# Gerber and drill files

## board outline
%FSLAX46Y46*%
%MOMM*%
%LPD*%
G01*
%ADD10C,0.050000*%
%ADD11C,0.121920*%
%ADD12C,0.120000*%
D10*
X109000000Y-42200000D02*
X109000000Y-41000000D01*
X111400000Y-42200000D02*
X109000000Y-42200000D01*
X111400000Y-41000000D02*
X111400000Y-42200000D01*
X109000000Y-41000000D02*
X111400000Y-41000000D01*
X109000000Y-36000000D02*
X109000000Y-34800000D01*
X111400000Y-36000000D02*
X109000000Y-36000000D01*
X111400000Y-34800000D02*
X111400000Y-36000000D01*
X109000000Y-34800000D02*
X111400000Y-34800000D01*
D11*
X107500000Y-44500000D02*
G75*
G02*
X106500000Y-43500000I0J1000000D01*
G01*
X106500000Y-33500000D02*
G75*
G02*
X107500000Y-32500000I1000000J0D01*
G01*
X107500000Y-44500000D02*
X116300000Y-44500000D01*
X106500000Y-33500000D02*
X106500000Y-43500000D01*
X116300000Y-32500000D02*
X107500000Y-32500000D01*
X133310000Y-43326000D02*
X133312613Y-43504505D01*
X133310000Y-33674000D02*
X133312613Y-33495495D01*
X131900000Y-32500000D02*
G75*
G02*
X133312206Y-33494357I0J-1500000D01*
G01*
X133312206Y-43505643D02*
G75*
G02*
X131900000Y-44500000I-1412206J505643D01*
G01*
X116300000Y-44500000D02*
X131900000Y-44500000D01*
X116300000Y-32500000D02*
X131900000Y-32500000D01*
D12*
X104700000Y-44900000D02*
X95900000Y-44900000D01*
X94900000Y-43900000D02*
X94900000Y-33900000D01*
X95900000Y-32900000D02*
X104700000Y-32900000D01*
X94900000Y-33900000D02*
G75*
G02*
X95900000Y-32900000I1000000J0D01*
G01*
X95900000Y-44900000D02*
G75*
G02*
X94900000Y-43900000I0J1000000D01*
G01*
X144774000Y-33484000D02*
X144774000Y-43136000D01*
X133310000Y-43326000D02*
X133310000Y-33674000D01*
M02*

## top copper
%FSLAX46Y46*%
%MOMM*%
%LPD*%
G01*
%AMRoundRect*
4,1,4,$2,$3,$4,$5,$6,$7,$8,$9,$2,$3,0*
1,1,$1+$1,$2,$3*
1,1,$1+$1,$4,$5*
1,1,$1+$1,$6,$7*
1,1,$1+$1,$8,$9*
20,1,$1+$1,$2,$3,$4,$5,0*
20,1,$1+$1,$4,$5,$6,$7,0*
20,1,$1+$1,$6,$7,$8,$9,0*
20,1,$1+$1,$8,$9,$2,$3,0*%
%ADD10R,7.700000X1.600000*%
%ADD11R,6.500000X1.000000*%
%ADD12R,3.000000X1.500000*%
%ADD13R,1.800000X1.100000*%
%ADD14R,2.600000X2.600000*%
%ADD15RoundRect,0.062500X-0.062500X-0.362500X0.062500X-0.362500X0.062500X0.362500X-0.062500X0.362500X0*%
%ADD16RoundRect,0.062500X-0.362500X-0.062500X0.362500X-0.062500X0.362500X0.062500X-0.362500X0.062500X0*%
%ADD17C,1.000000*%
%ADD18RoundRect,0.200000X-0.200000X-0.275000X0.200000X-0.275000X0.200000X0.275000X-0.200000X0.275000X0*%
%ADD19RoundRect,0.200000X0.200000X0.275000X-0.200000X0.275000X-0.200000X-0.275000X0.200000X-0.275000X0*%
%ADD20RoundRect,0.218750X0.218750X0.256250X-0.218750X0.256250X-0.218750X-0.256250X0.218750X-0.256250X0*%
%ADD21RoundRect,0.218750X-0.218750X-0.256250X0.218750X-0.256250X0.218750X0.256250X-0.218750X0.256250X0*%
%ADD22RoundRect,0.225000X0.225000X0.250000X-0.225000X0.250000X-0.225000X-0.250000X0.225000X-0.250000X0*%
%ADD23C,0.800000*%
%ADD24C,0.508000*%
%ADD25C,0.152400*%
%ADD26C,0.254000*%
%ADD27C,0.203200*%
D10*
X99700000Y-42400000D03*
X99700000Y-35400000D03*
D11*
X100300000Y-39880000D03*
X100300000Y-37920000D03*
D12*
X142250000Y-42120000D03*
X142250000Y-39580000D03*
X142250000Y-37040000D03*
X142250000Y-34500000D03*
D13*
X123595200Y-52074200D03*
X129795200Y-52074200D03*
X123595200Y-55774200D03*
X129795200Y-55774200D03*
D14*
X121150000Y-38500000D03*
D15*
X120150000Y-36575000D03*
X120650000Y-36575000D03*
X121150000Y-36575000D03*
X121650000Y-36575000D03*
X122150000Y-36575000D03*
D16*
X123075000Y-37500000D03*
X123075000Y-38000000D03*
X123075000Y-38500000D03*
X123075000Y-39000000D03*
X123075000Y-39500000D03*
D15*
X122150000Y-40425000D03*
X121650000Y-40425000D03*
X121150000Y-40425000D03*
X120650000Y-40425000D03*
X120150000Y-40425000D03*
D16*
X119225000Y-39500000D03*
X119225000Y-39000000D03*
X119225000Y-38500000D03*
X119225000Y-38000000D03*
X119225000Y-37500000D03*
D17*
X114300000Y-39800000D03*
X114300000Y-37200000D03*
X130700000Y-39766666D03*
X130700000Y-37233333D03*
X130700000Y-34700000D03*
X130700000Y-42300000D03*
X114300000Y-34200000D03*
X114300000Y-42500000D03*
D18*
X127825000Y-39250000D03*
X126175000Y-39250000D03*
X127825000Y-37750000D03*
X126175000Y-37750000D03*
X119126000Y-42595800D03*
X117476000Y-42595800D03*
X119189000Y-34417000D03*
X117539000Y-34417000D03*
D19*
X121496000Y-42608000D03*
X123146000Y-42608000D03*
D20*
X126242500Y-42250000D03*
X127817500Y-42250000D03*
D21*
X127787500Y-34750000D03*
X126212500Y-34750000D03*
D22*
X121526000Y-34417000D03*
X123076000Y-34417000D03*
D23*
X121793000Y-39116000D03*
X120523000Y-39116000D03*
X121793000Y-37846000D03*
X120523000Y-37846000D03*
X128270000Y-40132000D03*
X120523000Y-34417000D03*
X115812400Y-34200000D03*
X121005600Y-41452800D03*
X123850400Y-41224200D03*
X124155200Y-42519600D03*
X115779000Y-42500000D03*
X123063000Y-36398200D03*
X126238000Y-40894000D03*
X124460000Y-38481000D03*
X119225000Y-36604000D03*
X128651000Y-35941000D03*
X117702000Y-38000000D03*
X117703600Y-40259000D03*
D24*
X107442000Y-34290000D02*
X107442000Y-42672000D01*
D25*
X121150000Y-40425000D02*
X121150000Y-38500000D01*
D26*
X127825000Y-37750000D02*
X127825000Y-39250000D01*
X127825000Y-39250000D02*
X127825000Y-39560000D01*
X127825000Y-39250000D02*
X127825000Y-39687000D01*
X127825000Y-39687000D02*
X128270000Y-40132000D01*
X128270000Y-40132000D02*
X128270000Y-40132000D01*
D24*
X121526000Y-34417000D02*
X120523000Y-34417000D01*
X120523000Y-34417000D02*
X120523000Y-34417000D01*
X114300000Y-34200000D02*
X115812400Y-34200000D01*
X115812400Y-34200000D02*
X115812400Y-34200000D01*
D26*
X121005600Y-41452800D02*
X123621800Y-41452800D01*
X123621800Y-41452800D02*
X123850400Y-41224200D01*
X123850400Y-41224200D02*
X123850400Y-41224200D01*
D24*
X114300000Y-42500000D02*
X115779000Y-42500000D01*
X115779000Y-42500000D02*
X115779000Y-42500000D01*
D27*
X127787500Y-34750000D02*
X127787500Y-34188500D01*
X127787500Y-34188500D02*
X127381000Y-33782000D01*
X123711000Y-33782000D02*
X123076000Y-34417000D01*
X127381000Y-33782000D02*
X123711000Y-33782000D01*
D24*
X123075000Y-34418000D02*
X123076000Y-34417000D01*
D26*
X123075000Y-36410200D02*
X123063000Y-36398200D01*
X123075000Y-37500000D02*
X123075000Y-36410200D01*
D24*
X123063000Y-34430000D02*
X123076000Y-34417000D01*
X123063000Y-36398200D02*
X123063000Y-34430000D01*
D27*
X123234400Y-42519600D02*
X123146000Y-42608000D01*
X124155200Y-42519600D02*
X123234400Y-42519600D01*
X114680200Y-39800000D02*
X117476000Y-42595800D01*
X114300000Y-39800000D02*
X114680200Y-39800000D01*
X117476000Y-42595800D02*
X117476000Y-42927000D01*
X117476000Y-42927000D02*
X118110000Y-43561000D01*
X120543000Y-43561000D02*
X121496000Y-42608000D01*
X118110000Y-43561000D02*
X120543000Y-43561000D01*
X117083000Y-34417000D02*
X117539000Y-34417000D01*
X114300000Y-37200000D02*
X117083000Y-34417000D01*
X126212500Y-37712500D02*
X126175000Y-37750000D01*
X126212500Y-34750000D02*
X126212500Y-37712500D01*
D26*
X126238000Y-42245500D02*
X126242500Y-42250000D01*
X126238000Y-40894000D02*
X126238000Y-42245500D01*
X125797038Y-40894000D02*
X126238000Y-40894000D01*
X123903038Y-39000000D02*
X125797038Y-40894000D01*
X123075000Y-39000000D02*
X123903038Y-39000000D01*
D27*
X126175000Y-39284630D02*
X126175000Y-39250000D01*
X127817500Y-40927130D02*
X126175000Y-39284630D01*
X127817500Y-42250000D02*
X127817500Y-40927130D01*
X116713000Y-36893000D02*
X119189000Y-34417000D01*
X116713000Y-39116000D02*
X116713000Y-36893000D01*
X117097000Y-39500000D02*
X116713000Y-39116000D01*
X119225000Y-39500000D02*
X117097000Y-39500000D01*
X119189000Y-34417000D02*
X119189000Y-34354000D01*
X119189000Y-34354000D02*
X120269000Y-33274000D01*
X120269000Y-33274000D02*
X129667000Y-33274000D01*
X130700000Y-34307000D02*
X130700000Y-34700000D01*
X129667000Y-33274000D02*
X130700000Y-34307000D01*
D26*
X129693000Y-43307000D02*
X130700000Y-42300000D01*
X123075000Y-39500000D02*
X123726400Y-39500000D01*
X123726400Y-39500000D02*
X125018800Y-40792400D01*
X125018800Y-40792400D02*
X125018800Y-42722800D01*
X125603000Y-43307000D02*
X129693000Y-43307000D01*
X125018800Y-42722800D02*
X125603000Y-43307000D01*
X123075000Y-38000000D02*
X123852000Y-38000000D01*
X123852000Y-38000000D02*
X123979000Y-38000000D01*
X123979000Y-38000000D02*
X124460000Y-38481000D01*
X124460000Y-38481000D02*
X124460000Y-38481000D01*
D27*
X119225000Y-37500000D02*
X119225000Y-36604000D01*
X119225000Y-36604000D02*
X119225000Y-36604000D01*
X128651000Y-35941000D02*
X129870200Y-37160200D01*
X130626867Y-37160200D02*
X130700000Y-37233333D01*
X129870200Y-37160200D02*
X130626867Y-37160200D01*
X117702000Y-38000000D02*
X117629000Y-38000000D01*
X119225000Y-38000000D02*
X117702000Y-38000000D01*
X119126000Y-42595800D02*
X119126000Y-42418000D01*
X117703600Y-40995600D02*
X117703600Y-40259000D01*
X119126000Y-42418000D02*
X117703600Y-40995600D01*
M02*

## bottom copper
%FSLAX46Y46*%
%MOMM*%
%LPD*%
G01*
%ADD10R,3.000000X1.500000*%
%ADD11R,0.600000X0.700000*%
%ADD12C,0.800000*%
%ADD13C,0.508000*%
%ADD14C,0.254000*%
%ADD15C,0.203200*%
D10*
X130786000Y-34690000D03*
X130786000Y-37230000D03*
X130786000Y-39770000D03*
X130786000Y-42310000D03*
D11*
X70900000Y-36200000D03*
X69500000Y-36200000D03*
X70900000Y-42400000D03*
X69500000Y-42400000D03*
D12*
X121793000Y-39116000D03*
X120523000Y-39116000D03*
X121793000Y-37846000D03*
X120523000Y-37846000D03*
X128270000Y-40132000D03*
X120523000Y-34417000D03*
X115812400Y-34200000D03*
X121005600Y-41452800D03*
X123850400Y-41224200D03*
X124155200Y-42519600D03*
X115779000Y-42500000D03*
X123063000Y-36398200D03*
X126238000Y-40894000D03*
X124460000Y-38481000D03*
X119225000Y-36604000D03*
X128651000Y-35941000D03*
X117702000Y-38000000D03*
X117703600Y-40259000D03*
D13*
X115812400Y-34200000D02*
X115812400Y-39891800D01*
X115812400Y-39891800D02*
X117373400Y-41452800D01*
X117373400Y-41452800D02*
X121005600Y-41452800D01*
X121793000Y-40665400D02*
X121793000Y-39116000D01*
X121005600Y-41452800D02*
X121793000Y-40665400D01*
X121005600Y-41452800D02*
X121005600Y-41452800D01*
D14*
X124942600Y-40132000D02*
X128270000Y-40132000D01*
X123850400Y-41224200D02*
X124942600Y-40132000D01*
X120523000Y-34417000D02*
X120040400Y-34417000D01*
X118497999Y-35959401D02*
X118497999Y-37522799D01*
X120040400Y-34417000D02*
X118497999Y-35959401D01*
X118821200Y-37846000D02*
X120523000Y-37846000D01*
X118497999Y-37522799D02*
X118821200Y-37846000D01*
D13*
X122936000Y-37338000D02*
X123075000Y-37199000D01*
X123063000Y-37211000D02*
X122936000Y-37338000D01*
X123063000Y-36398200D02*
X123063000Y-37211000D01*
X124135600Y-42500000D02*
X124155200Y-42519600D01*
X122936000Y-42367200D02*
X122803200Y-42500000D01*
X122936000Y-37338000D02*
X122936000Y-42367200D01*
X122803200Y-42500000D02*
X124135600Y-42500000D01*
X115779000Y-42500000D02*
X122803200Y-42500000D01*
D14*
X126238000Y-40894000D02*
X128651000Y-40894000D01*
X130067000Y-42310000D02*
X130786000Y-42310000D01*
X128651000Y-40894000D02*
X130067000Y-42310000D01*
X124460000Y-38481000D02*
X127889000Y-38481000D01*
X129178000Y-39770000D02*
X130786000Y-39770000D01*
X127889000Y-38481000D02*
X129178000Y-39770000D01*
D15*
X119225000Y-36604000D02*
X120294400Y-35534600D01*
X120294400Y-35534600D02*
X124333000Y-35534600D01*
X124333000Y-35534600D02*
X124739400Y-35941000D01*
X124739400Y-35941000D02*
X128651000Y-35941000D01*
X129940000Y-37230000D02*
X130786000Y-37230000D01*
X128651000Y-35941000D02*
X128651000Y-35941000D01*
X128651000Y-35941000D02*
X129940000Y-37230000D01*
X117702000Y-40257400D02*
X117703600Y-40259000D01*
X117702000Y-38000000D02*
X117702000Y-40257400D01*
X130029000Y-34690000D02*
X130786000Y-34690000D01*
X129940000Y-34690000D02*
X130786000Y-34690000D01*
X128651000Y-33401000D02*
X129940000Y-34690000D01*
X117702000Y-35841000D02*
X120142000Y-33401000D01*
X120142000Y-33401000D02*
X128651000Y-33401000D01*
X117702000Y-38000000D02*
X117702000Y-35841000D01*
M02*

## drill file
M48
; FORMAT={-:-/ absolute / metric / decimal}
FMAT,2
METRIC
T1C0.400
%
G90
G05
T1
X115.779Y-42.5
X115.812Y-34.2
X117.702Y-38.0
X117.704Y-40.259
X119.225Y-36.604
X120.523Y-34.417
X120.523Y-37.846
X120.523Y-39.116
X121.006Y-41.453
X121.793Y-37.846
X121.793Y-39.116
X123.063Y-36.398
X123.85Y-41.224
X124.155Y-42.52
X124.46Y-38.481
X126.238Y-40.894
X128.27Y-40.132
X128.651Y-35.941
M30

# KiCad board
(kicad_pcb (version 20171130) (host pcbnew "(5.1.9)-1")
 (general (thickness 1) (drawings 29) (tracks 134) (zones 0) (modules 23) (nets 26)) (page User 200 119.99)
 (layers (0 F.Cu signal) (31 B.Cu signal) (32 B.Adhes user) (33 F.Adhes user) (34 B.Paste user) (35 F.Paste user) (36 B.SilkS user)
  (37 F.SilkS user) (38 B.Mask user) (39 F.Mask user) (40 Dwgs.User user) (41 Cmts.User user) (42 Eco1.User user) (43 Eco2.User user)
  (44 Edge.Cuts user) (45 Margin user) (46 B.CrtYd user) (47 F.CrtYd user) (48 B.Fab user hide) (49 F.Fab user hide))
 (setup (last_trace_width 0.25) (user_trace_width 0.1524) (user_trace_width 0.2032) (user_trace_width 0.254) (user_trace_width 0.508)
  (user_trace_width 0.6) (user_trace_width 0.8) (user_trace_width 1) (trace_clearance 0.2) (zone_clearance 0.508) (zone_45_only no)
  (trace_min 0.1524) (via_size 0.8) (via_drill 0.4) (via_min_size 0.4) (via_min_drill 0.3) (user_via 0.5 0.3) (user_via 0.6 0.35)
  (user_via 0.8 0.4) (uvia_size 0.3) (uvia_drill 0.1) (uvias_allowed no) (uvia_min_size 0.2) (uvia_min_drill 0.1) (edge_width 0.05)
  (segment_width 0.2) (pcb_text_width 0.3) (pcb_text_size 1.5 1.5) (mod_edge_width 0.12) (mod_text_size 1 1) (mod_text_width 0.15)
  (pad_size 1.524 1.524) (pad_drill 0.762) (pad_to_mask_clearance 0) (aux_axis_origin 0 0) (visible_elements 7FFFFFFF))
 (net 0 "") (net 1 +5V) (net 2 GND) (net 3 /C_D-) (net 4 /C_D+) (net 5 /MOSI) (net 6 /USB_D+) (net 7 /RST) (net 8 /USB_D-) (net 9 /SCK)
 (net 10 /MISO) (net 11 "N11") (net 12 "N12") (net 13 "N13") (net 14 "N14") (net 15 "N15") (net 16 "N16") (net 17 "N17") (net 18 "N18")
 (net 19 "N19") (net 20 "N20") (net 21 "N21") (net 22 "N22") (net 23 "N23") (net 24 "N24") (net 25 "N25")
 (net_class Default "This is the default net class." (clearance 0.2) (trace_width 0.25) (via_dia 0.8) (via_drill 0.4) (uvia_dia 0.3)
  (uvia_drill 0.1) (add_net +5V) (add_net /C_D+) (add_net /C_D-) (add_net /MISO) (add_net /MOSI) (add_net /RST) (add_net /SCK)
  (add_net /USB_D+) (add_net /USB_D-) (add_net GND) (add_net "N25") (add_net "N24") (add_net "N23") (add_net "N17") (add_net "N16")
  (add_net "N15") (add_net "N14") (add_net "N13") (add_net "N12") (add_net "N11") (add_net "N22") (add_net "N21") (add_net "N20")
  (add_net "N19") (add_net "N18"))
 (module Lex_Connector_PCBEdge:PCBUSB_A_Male (layer F.Cu) (at 100.7 38.9 180)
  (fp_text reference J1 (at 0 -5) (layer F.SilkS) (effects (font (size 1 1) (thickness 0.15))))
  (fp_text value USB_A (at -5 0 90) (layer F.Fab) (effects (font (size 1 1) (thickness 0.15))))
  (fp_line (start -4 -6) (end 4.8 -6) (layer Edge.Cuts) (width 0.12))
  (fp_line (start 5.8 -5) (end 5.8 5) (layer Edge.Cuts) (width 0.12))
  (fp_line (start 4.8 6) (end -4 6) (layer Edge.Cuts) (width 0.12))
  (fp_arc (start 4.8 5) (end 4.8 6) (angle -90) (layer Edge.Cuts) (width 0.12))
  (fp_arc (start 4.8 -5) (end 5.8 -5) (angle -90) (layer Edge.Cuts) (width 0.12))
  (pad 1 connect rect (at 1 -3.5 180) (size 7.7 1.6) (layers F.Cu F.Mask) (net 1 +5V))
  (pad 4 connect rect (at 1 3.5 180) (size 7.7 1.6) (layers F.Cu F.Mask) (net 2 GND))
  (pad 2 connect rect (at 0.4 -0.98 180) (size 6.5 1) (layers F.Cu F.Mask) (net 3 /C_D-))
  (pad 3 connect rect (at 0.4 0.98 180) (size 6.5 1) (layers F.Cu F.Mask) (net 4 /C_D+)))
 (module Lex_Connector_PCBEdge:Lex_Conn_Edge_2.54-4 (layer F.Cu) (at 139.964 38.31)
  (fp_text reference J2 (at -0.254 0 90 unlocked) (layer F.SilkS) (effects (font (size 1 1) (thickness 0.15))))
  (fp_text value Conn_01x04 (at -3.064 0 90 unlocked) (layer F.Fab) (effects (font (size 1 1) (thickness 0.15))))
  (fp_line (start 4.81 -4.826) (end 4.81 4.826) (layer Edge.Cuts) (width 0.12))
  (pad 4 smd rect (at 2.286 3.81 270) (size 1.5 3) (layers F.Cu F.Paste F.Mask) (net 1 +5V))
  (pad 3 smd rect (at 2.286 1.27 270) (size 1.5 3) (layers F.Cu F.Paste F.Mask) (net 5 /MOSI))
  (pad 2 smd rect (at 2.286 -1.27 270) (size 1.5 3) (layers F.Cu F.Paste F.Mask) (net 2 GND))
  (pad 1 smd rect (at 2.286 -3.81 270) (size 1.5 3) (layers F.Cu F.Paste F.Mask) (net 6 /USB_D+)))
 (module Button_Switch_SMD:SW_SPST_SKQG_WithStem (layer F.Cu) (at 126.6952 53.9242 180)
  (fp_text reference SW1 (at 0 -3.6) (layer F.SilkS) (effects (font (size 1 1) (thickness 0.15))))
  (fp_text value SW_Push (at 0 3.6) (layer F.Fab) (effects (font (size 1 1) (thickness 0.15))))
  (pad 2 smd rect (at 3.1 1.85 180) (size 1.8 1.1) (layers F.Cu F.Paste F.Mask) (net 2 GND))
  (pad 2 smd rect (at -3.1 1.85 180) (size 1.8 1.1) (layers F.Cu F.Paste F.Mask) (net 2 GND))
  (pad 1 smd rect (at 3.1 -1.85 180) (size 1.8 1.1) (layers F.Cu F.Paste F.Mask) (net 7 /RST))
  (pad 1 smd rect (at -3.1 -1.85 180) (size 1.8 1.1) (layers F.Cu F.Paste F.Mask) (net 7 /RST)))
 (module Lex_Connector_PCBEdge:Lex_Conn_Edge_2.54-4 (layer B.Cu) (at 128.5 38.5)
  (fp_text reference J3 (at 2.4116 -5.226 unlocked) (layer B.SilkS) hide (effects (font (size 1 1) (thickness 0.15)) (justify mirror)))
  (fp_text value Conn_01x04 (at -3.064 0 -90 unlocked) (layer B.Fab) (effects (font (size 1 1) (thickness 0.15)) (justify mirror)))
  (fp_line (start 4.81 4.826) (end 4.81 -4.826) (layer Edge.Cuts) (width 0.12))
  (pad 4 smd rect (at 2.286 -3.81 90) (size 1.5 3) (layers B.Cu B.Paste B.Mask) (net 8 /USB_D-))
  (pad 3 smd rect (at 2.286 -1.27 90) (size 1.5 3) (layers B.Cu B.Paste B.Mask) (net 7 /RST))
  (pad 2 smd rect (at 2.286 1.27 90) (size 1.5 3) (layers B.Cu B.Paste B.Mask) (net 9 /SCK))
  (pad 1 smd rect (at 2.286 3.81 90) (size 1.5 3) (layers B.Cu B.Paste B.Mask) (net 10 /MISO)))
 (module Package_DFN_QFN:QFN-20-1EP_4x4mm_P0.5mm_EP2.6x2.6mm (layer F.Cu) (at 121.15 38.5)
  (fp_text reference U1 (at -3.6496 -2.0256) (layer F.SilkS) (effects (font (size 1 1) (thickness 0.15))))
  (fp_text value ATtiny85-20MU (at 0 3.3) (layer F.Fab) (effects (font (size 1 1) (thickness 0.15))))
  (pad "" smd roundrect (at 0.65 0.65) (size 1.05 1.05) (layers F.Paste) (roundrect_rratio 0.238095))
  (pad "" smd roundrect (at 0.65 -0.65) (size 1.05 1.05) (layers F.Paste) (roundrect_rratio 0.238095))
  (pad "" smd roundrect (at -0.65 0.65) (size 1.05 1.05) (layers F.Paste) (roundrect_rratio 0.238095))
  (pad "" smd roundrect (at -0.65 -0.65) (size 1.05 1.05) (layers F.Paste) (roundrect_rratio 0.238095))
  (pad 21 smd rect (at 0 0) (size 2.6 2.6) (layers F.Cu F.Mask) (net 2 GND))
  (pad 20 smd roundrect (at -1 -1.925) (size 0.25 0.85) (layers F.Cu F.Paste F.Mask) (roundrect_rratio 0.25) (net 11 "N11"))
  (pad 19 smd roundrect (at -0.5 -1.925) (size 0.25 0.85) (layers F.Cu F.Paste F.Mask) (roundrect_rratio 0.25) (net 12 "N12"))
  (pad 18 smd roundrect (at 0 -1.925) (size 0.25 0.85) (layers F.Cu F.Paste F.Mask) (roundrect_rratio 0.25) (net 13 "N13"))
  (pad 17 smd roundrect (at 0.5 -1.925) (size 0.25 0.85) (layers F.Cu F.Paste F.Mask) (roundrect_rratio 0.25) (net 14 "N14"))
  (pad 16 smd roundrect (at 1 -1.925) (size 0.25 0.85) (layers F.Cu F.Paste F.Mask) (roundrect_rratio 0.25) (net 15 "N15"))
  (pad 15 smd roundrect (at 1.925 -1) (size 0.85 0.25) (layers F.Cu F.Paste F.Mask) (roundrect_rratio 0.25) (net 1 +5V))
  (pad 14 smd roundrect (at 1.925 -0.5) (size 0.85 0.25) (layers F.Cu F.Paste F.Mask) (roundrect_rratio 0.25) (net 9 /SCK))
  (pad 13 smd roundrect (at 1.925 0) (size 0.85 0.25) (layers F.Cu F.Paste F.Mask) (roundrect_rratio 0.25) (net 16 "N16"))
  (pad 12 smd roundrect (at 1.925 0.5) (size 0.85 0.25) (layers F.Cu F.Paste F.Mask) (roundrect_rratio 0.25) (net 10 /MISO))
  (pad 11 smd roundrect (at 1.925 1) (size 0.85 0.25) (layers F.Cu F.Paste F.Mask) (roundrect_rratio 0.25) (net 5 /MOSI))
  (pad 10 smd roundrect (at 1 1.925) (size 0.25 0.85) (layers F.Cu F.Paste F.Mask) (roundrect_rratio 0.25) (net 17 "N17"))
  (pad 9 smd roundrect (at 0.5 1.925) (size 0.25 0.85) (layers F.Cu F.Paste F.Mask) (roundrect_rratio 0.25) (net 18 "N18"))
  (pad 8 smd roundrect (at 0 1.925) (size 0.25 0.85) (layers F.Cu F.Paste F.Mask) (roundrect_rratio 0.25) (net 2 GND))
  (pad 7 smd roundrect (at -0.5 1.925) (size 0.25 0.85) (layers F.Cu F.Paste F.Mask) (roundrect_rratio 0.25) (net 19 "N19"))
  (pad 6 smd roundrect (at -1 1.925) (size 0.25 0.85) (layers F.Cu F.Paste F.Mask) (roundrect_rratio 0.25) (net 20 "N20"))
  (pad 5 smd roundrect (at -1.925 1) (size 0.85 0.25) (layers F.Cu F.Paste F.Mask) (roundrect_rratio 0.25) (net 6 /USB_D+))
  (pad 4 smd roundrect (at -1.925 0.5) (size 0.85 0.25) (layers F.Cu F.Paste F.Mask) (roundrect_rratio 0.25) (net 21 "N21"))
  (pad 3 smd roundrect (at -1.925 0) (size 0.85 0.25) (layers F.Cu F.Paste F.Mask) (roundrect_rratio 0.25) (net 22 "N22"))
  (pad 2 smd roundrect (at -1.925 -0.5) (size 0.85 0.25) (layers F.Cu F.Paste F.Mask) (roundrect_rratio 0.25) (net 8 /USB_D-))
  (pad 1 smd roundrect (at -1.925 -1) (size 0.85 0.25) (layers F.Cu F.Paste F.Mask) (roundrect_rratio 0.25) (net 7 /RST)))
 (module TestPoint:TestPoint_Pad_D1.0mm (layer F.Cu) (at 114.3 39.8)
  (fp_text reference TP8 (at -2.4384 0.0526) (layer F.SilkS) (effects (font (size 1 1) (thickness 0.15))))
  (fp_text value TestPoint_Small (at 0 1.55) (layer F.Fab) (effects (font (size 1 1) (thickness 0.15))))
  (pad 1 smd circle (at 0 0) (size 1 1) (layers F.Cu F.Mask) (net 3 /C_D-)))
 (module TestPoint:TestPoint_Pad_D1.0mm (layer F.Cu) (at 114.3 37.2)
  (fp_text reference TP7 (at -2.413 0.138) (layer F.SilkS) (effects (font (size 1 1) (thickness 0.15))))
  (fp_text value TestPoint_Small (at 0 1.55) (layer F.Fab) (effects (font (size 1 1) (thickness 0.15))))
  (pad 1 smd circle (at 0 0) (size 1 1) (layers F.Cu F.Mask) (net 4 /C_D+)))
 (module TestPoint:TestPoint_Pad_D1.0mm (layer F.Cu) (at 130.7 39.766666)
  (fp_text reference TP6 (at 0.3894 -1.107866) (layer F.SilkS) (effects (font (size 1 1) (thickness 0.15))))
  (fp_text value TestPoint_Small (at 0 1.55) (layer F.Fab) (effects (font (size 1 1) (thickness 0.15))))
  (pad 1 smd circle (at 0 0) (size 1 1) (layers F.Cu F.Mask) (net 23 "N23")))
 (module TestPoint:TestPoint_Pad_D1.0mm (layer F.Cu) (at 130.7 37.233333)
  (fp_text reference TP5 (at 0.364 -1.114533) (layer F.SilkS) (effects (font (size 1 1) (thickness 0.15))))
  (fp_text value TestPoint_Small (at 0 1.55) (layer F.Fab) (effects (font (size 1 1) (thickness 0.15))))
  (pad 1 smd circle (at 0 0) (size 1 1) (layers F.Cu F.Mask) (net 7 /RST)))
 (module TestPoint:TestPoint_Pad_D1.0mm (layer F.Cu) (at 130.7 34.7)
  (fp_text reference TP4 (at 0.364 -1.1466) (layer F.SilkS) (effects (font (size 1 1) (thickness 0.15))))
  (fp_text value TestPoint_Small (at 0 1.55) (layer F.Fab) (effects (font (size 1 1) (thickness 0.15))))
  (pad 1 smd circle (at 0 0) (size 1 1) (layers F.Cu F.Mask) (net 6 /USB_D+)))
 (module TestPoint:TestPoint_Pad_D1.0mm (layer F.Cu) (at 130.7 42.3)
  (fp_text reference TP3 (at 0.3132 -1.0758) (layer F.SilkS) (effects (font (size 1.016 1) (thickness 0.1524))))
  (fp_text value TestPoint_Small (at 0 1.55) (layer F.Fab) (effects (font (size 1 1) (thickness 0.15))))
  (pad 1 smd circle (at 0 0) (size 1 1) (layers F.Cu F.Mask) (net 5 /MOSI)))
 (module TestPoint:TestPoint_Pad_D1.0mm (layer F.Cu) (at 114.3 34.2)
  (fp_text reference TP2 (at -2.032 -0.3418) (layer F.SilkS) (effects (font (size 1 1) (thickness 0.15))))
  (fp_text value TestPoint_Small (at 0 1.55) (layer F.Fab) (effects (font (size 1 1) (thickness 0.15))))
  (pad 1 smd circle (at 0 0) (size 1 1) (layers F.Cu F.Mask) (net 2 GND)))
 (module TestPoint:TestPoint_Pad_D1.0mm (layer F.Cu) (at 114.3 42.5)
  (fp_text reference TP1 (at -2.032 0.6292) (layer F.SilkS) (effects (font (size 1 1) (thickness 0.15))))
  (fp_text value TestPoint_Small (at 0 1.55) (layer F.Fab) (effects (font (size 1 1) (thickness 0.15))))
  (pad 1 smd circle (at 0 0) (size 1 1) (layers F.Cu F.Mask) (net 1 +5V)))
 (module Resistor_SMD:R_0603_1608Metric (layer F.Cu) (at 127 39.25)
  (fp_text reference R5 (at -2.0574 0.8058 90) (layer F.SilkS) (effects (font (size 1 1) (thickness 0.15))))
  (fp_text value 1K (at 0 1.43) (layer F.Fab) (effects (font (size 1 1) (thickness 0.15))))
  (pad 2 smd roundrect (at 0.825 0) (size 0.8 0.95) (layers F.Cu F.Paste F.Mask) (roundrect_rratio 0.25) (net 2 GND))
  (pad 1 smd roundrect (at -0.825 0) (size 0.8 0.95) (layers F.Cu F.Paste F.Mask) (roundrect_rratio 0.25) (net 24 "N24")))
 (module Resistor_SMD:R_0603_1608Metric (layer F.Cu) (at 127 37.75)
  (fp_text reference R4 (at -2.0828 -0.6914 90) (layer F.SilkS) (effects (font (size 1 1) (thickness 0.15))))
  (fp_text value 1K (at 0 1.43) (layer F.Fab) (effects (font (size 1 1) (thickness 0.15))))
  (pad 2 smd roundrect (at 0.825 0) (size 0.8 0.95) (layers F.Cu F.Paste F.Mask) (roundrect_rratio 0.25) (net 2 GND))
  (pad 1 smd roundrect (at -0.825 0) (size 0.8 0.95) (layers F.Cu F.Paste F.Mask) (roundrect_rratio 0.25) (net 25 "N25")))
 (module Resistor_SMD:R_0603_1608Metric (layer F.Cu) (at 118.301 42.5958)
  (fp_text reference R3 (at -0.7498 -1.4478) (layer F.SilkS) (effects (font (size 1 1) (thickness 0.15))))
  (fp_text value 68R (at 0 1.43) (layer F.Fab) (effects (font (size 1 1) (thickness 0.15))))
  (pad 2 smd roundrect (at 0.825 0) (size 0.8 0.95) (layers F.Cu F.Paste F.Mask) (roundrect_rratio 0.25) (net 8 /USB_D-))
  (pad 1 smd roundrect (at -0.825 0) (size 0.8 0.95) (layers F.Cu F.Paste F.Mask) (roundrect_rratio 0.25) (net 3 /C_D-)))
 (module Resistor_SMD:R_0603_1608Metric (layer F.Cu) (at 118.364 34.417)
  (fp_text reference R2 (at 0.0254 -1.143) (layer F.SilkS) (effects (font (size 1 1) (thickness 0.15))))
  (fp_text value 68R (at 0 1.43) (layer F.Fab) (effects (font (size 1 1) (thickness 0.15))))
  (pad 2 smd roundrect (at 0.825 0) (size 0.8 0.95) (layers F.Cu F.Paste F.Mask) (roundrect_rratio 0.25) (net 6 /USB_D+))
  (pad 1 smd roundrect (at -0.825 0) (size 0.8 0.95) (layers F.Cu F.Paste F.Mask) (roundrect_rratio 0.25) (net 4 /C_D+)))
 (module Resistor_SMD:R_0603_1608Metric (layer F.Cu) (at 122.321 42.608 180)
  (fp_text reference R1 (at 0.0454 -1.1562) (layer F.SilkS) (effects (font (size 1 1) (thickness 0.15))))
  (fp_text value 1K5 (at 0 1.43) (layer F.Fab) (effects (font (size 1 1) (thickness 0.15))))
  (pad 2 smd roundrect (at 0.825 0 180) (size 0.8 0.95) (layers F.Cu F.Paste F.Mask) (roundrect_rratio 0.25) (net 3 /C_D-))
  (pad 1 smd roundrect (at -0.825 0 180) (size 0.8 0.95) (layers F.Cu F.Paste F.Mask) (roundrect_rratio 0.25) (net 1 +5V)))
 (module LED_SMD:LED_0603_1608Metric (layer F.Cu) (at 127.03 42.25 180)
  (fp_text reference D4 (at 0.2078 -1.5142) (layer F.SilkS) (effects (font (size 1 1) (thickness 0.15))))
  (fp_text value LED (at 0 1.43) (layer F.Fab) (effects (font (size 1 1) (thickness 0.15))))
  (pad 2 smd roundrect (at 0.7875 0 180) (size 0.875 0.95) (layers F.Cu F.Paste F.Mask) (roundrect_rratio 0.25) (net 10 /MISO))
  (pad 1 smd roundrect (at -0.7875 0 180) (size 0.875 0.95) (layers F.Cu F.Paste F.Mask) (roundrect_rratio 0.25) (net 24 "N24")))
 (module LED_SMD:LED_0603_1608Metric (layer F.Cu) (at 127 34.75)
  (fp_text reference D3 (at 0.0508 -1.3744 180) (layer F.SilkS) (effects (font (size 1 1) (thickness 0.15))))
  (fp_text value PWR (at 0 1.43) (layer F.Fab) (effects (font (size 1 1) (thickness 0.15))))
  (pad 2 smd roundrect (at 0.7875 0) (size 0.875 0.95) (layers F.Cu F.Paste F.Mask) (roundrect_rratio 0.25) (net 1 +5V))
  (pad 1 smd roundrect (at -0.7875 0) (size 0.875 0.95) (layers F.Cu F.Paste F.Mask) (roundrect_rratio 0.25) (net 25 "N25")))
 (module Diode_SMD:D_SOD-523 (layer B.Cu) (at 70.2 36.2 180)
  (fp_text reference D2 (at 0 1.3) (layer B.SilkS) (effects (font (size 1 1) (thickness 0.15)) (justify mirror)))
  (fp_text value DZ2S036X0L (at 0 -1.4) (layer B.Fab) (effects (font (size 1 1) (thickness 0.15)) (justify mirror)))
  (pad 1 smd rect (at -0.7 0) (size 0.6 0.7) (layers B.Cu B.Paste B.Mask) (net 4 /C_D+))
  (pad 2 smd rect (at 0.7 0) (size 0.6 0.7) (layers B.Cu B.Paste B.Mask) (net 2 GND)))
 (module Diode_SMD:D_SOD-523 (layer B.Cu) (at 70.2 42.4 180)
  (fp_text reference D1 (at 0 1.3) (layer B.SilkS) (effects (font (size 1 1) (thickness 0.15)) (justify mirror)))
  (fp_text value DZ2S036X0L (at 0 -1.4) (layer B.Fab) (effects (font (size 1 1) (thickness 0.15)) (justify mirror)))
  (pad 1 smd rect (at -0.7 0) (size 0.6 0.7) (layers B.Cu B.Paste B.Mask) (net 3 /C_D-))
  (pad 2 smd rect (at 0.7 0) (size 0.6 0.7) (layers B.Cu B.Paste B.Mask) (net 2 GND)))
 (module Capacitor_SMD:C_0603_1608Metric (layer F.Cu) (at 122.301 34.417 180)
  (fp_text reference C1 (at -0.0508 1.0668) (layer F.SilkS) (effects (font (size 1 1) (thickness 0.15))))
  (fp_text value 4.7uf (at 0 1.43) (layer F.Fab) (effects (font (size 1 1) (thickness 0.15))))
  (pad 2 smd roundrect (at 0.775 0 180) (size 0.9 0.95) (layers F.Cu F.Paste F.Mask) (roundrect_rratio 0.25) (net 2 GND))
  (pad 1 smd roundrect (at -0.775 0 180) (size 0.9 0.95) (layers F.Cu F.Paste F.Mask) (roundrect_rratio 0.25) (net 1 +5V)))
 (gr_line (start 109 42.2) (end 109 41) (layer Edge.Cuts) (width 0.05))
 (gr_line (start 111.4 42.2) (end 109 42.2) (layer Edge.Cuts) (width 0.05))
 (gr_line (start 111.4 41) (end 111.4 42.2) (layer Edge.Cuts) (width 0.05))
 (gr_line (start 109 41) (end 111.4 41) (layer Edge.Cuts) (width 0.05))
 (gr_line (start 109 36) (end 109 34.8) (layer Edge.Cuts) (width 0.05))
 (gr_line (start 111.4 36) (end 109 36) (layer Edge.Cuts) (width 0.05))
 (gr_line (start 111.4 34.8) (end 111.4 36) (layer Edge.Cuts) (width 0.05))
 (gr_line (start 109 34.8) (end 111.4 34.8) (layer Edge.Cuts) (width 0.05))
 (gr_arc (start 107.5 43.5) (end 106.5 43.5) (angle -90) (layer Edge.Cuts) (width 0.12192))
 (gr_arc (start 107.5 33.5) (end 107.5 32.5) (angle -90) (layer Edge.Cuts) (width 0.12192))
 (gr_line (start 107.5 44.5) (end 116.3 44.5) (layer Edge.Cuts) (width 0.12192))
 (gr_line (start 106.5 33.5) (end 106.5 43.5) (layer Edge.Cuts) (width 0.12192))
 (gr_line (start 116.3 32.5) (end 107.5 32.5) (layer Edge.Cuts) (width 0.12192))
 (gr_line (start 133.31 43.326) (end 133.312613 43.504505) (layer Edge.Cuts) (width 0.12192))
 (gr_line (start 133.31 33.674) (end 133.312613 33.495495) (layer Edge.Cuts) (width 0.12192))
 (gr_arc (start 131.9 34) (end 131.9 32.5) (angle 70.3) (layer Edge.Cuts) (width 0.12192))
 (gr_arc (start 131.9 43) (end 131.9 44.5) (angle -70.3) (layer Edge.Cuts) (width 0.12192))
 (gr_line (start 116.3 44.5) (end 131.9 44.5) (layer Edge.Cuts) (width 0.12192))
 (gr_line (start 116.3 32.5) (end 131.9 32.5) (layer Edge.Cuts) (width 0.12192))
 (segment (start 107.442 34.29) (end 107.442 42.672) (width 0.508) (layer F.Cu) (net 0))
 (via (at 121.793 39.116) (size 0.8) (drill 0.4) (layers F.Cu B.Cu) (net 2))
 (via (at 120.523 39.116) (size 0.8) (drill 0.4) (layers F.Cu B.Cu) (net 2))
 (via (at 121.793 37.846) (size 0.8) (drill 0.4) (layers F.Cu B.Cu) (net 2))
 (via (at 120.523 37.846) (size 0.8) (drill 0.4) (layers F.Cu B.Cu) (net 2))
 (segment (start 121.15 40.425) (end 121.15 38.5) (width 0.1524) (layer F.Cu) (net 2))
 (segment (start 127.825 37.75) (end 127.825 39.25) (width 0.254) (layer F.Cu) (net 2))
 (segment (start 127.825 39.25) (end 127.825 39.56) (width 0.254) (layer F.Cu) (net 2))
 (segment (start 127.825 39.25) (end 127.825 39.687) (width 0.254) (layer F.Cu) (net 2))
 (segment (start 127.825 39.687) (end 128.27 40.132) (width 0.254) (layer F.Cu) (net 2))
 (segment (start 128.27 40.132) (end 128.27 40.132) (width 0.254) (layer F.Cu) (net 2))
 (via (at 128.27 40.132) (size 0.8) (drill 0.4) (layers F.Cu B.Cu) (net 2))
 (segment (start 121.526 34.417) (end 120.523 34.417) (width 0.508) (layer F.Cu) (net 2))
 (segment (start 120.523 34.417) (end 120.523 34.417) (width 0.508) (layer F.Cu) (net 2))
 (via (at 120.523 34.417) (size 0.8) (drill 0.4) (layers F.Cu B.Cu) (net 2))
 (segment (start 114.3 34.2) (end 115.8124 34.2) (width 0.508) (layer F.Cu) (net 2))
 (segment (start 115.8124 34.2) (end 115.8124 34.2) (width 0.508) (layer F.Cu) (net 2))
 (via (at 115.8124 34.2) (size 0.8) (drill 0.4) (layers F.Cu B.Cu) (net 2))
 (segment (start 115.8124 34.2) (end 115.8124 39.8918) (width 0.508) (layer B.Cu) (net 2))
 (segment (start 115.8124 39.8918) (end 117.3734 41.4528) (width 0.508) (layer B.Cu) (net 2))
 (segment (start 117.3734 41.4528) (end 121.0056 41.4528) (width 0.508) (layer B.Cu) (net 2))
 (segment (start 121.793 40.6654) (end 121.793 39.116) (width 0.508) (layer B.Cu) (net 2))
 (segment (start 121.0056 41.4528) (end 121.793 40.6654) (width 0.508) (layer B.Cu) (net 2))
 (segment (start 121.0056 41.4528) (end 121.0056 41.4528) (width 0.508) (layer B.Cu) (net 2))
 (via (at 121.0056 41.4528) (size 0.8) (drill 0.4) (layers F.Cu B.Cu) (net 2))
 (segment (start 121.0056 41.4528) (end 123.6218 41.4528) (width 0.254) (layer F.Cu) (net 2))
 (segment (start 123.6218 41.4528) (end 123.8504 41.2242) (width 0.254) (layer F.Cu) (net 2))
 (segment (start 123.8504 41.2242) (end 123.8504 41.2242) (width 0.254) (layer F.Cu) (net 2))
 (via (at 123.8504 41.2242) (size 0.8) (drill 0.4) (layers F.Cu B.Cu) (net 2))
 (segment (start 124.9426 40.132) (end 128.27 40.132) (width 0.254) (layer B.Cu) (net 2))
 (segment (start 123.8504 41.2242) (end 124.9426 40.132) (width 0.254) (layer B.Cu) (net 2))
 (segment (start 120.523 34.417) (end 120.0404 34.417) (width 0.254) (layer B.Cu) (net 2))
 (segment (start 118.497999 35.959401) (end 118.497999 37.522799) (width 0.254) (layer B.Cu) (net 2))
 (segment (start 120.0404 34.417) (end 118.497999 35.959401) (width 0.254) (layer B.Cu) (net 2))
 (segment (start 118.8212 37.846) (end 120.523 37.846) (width 0.254) (layer B.Cu) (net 2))
 (segment (start 118.497999 37.522799) (end 118.8212 37.846) (width 0.254) (layer B.Cu) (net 2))
 (via (at 124.1552 42.5196) (size 0.8) (drill 0.4) (layers F.Cu B.Cu) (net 1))
 (segment (start 114.3 42.5) (end 115.779 42.5) (width 0.508) (layer F.Cu) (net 1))
 (segment (start 115.779 42.5) (end 115.779 42.5) (width 0.508) (layer F.Cu) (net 1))
 (via (at 115.779 42.5) (size 0.8) (drill 0.4) (layers F.Cu B.Cu) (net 1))
 (segment (start 127.7875 34.75) (end 127.7875 34.1885) (width 0.2032) (layer F.Cu) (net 1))
 (segment (start 127.7875 34.1885) (end 127.381 33.782) (width 0.2032) (layer F.Cu) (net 1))
 (segment (start 123.711 33.782) (end 123.076 34.417) (width 0.2032) (layer F.Cu) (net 1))
 (segment (start 127.381 33.782) (end 123.711 33.782) (width 0.2032) (layer F.Cu) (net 1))
 (segment (start 123.075 34.418) (end 123.076 34.417) (width 0.508) (layer F.Cu) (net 1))
 (via (at 123.063 36.3982) (size 0.8) (drill 0.4) (layers F.Cu B.Cu) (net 1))
 (segment (start 122.936 37.338) (end 123.075 37.199) (width 0.508) (layer B.Cu) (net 1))
 (segment (start 123.075 36.4102) (end 123.063 36.3982) (width 0.254) (layer F.Cu) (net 1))
 (segment (start 123.075 37.5) (end 123.075 36.4102) (width 0.254) (layer F.Cu) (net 1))
 (segment (start 123.063 34.43) (end 123.076 34.417) (width 0.508) (layer F.Cu) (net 1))
 (segment (start 123.063 36.3982) (end 123.063 34.43) (width 0.508) (layer F.Cu) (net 1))
 (segment (start 123.063 37.211) (end 122.936 37.338) (width 0.508) (layer B.Cu) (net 1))
 (segment (start 123.063 36.3982) (end 123.063 37.211) (width 0.508) (layer B.Cu) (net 1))
 (segment (start 124.1356 42.5) (end 124.1552 42.5196) (width 0.508) (layer B.Cu) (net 1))
 (segment (start 122.936 42.3672) (end 122.8032 42.5) (width 0.508) (layer B.Cu) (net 1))
 (segment (start 122.936 37.338) (end 122.936 42.3672) (width 0.508) (layer B.Cu) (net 1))
 (segment (start 122.8032 42.5) (end 124.1356 42.5) (width 0.508) (layer B.Cu) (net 1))
 (segment (start 115.779 42.5) (end 122.8032 42.5) (width 0.508) (layer B.Cu) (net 1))
 (segment (start 123.2344 42.5196) (end 123.146 42.608) (width 0.2032) (layer F.Cu) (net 1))
 (segment (start 124.1552 42.5196) (end 123.2344 42.5196) (width 0.2032) (layer F.Cu) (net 1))
 (segment (start 114.6802 39.8) (end 117.476 42.5958) (width 0.2032) (layer F.Cu) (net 3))
 (segment (start 114.3 39.8) (end 114.6802 39.8) (width 0.2032) (layer F.Cu) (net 3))
 (segment (start 117.476 42.5958) (end 117.476 42.927) (width 0.2032) (layer F.Cu) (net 3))
 (segment (start 117.476 42.927) (end 118.11 43.561) (width 0.2032) (layer F.Cu) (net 3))
 (segment (start 120.543 43.561) (end 121.496 42.608) (width 0.2032) (layer F.Cu) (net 3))
 (segment (start 118.11 43.561) (end 120.543 43.561) (width 0.2032) (layer F.Cu) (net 3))
 (segment (start 117.083 34.417) (end 117.539 34.417) (width 0.2032) (layer F.Cu) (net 4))
 (segment (start 114.3 37.2) (end 117.083 34.417) (width 0.2032) (layer F.Cu) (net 4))
 (segment (start 126.2125 37.7125) (end 126.175 37.75) (width 0.2032) (layer F.Cu) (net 25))
 (segment (start 126.2125 34.75) (end 126.2125 37.7125) (width 0.2032) (layer F.Cu) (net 25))
 (via (at 126.238 40.894) (size 0.8) (drill 0.4) (layers F.Cu B.Cu) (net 10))
 (segment (start 126.238 42.2455) (end 126.2425 42.25) (width 0.254) (layer F.Cu) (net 10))
 (segment (start 126.238 40.894) (end 126.238 42.2455) (width 0.254) (layer F.Cu) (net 10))
 (segment (start 126.238 40.894) (end 128.651 40.894) (width 0.254) (layer B.Cu) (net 10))
 (segment (start 130.067 42.31) (end 130.786 42.31) (width 0.254) (layer B.Cu) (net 10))
 (segment (start 128.651 40.894) (end 130.067 42.31) (width 0.254) (layer B.Cu) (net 10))
 (segment (start 125.797038 40.894) (end 126.238 40.894) (width 0.254) (layer F.Cu) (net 10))
 (segment (start 123.903038 39) (end 125.797038 40.894) (width 0.254) (layer F.Cu) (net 10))
 (segment (start 123.075 39) (end 123.903038 39) (width 0.254) (layer F.Cu) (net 10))
 (segment (start 126.175 39.28463) (end 126.175 39.25) (width 0.2032) (layer F.Cu) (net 24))
 (segment (start 127.8175 40.92713) (end 126.175 39.28463) (width 0.2032) (layer F.Cu) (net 24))
 (segment (start 127.8175 42.25) (end 127.8175 40.92713) (width 0.2032) (layer F.Cu) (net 24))
 (segment (start 116.713 36.893) (end 119.189 34.417) (width 0.2032) (layer F.Cu) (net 6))
 (segment (start 116.713 39.116) (end 116.713 36.893) (width 0.2032) (layer F.Cu) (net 6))
 (segment (start 117.097 39.5) (end 116.713 39.116) (width 0.2032) (layer F.Cu) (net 6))
 (segment (start 119.225 39.5) (end 117.097 39.5) (width 0.2032) (layer F.Cu) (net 6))
 (segment (start 119.189 34.417) (end 119.189 34.354) (width 0.2032) (layer F.Cu) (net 6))
 (segment (start 119.189 34.354) (end 120.269 33.274) (width 0.2032) (layer F.Cu) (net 6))
 (segment (start 120.269 33.274) (end 129.667 33.274) (width 0.2032) (layer F.Cu) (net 6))
 (segment (start 130.7 34.307) (end 130.7 34.7) (width 0.2032) (layer F.Cu) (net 6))
 (segment (start 129.667 33.274) (end 130.7 34.307) (width 0.2032) (layer F.Cu) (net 6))
 (segment (start 129.693 43.307) (end 130.7 42.3) (width 0.254) (layer F.Cu) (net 5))
 (segment (start 123.075 39.5) (end 123.7264 39.5) (width 0.254) (layer F.Cu) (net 5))
 (segment (start 123.7264 39.5) (end 125.0188 40.7924) (width 0.254) (layer F.Cu) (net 5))
 (segment (start 125.0188 40.7924) (end 125.0188 42.7228) (width 0.254) (layer F.Cu) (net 5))
 (segment (start 125.603 43.307) (end 129.693 43.307) (width 0.254) (layer F.Cu) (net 5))
 (segment (start 125.0188 42.7228) (end 125.603 43.307) (width 0.254) (layer F.Cu) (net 5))
 (segment (start 123.075 38) (end 123.852 38) (width 0.254) (layer F.Cu) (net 9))
 (segment (start 123.852 38) (end 123.979 38) (width 0.254) (layer F.Cu) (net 9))
 (segment (start 123.979 38) (end 124.46 38.481) (width 0.254) (layer F.Cu) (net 9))
 (segment (start 124.46 38.481) (end 124.46 38.481) (width 0.254) (layer F.Cu) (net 9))
 (via (at 124.46 38.481) (size 0.8) (drill 0.4) (layers F.Cu B.Cu) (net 9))
 (segment (start 124.46 38.481) (end 127.889 38.481) (width 0.254) (layer B.Cu) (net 9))
 (segment (start 129.178 39.77) (end 130.786 39.77) (width 0.254) (layer B.Cu) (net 9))
 (segment (start 127.889 38.481) (end 129.178 39.77) (width 0.254) (layer B.Cu) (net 9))
 (segment (start 119.225 37.5) (end 119.225 36.604) (width 0.2032) (layer F.Cu) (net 7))
 (segment (start 119.225 36.604) (end 119.225 36.604) (width 0.2032) (layer F.Cu) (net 7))
 (via (at 119.225 36.604) (size 0.8) (drill 0.4) (layers F.Cu B.Cu) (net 7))
 (segment (start 119.225 36.604) (end 120.2944 35.5346) (width 0.2032) (layer B.Cu) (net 7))
 (segment (start 120.2944 35.5346) (end 124.333 35.5346) (width 0.2032) (layer B.Cu) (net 7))
 (segment (start 124.333 35.5346) (end 124.7394 35.941) (width 0.2032) (layer B.Cu) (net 7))
 (segment (start 124.7394 35.941) (end 128.651 35.941) (width 0.2032) (layer B.Cu) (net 7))
 (segment (start 129.94 37.23) (end 130.786 37.23) (width 0.2032) (layer B.Cu) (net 7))
 (segment (start 128.651 35.941) (end 128.651 35.941) (width 0.2032) (layer B.Cu) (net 7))
 (segment (start 128.651 35.941) (end 129.94 37.23) (width 0.2032) (layer B.Cu) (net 7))
 (via (at 128.651 35.941) (size 0.8) (drill 0.4) (layers F.Cu B.Cu) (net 7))
 (segment (start 128.651 35.941) (end 129.8702 37.1602) (width 0.2032) (layer F.Cu) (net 7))
 (segment (start 130.626867 37.1602) (end 130.7 37.233333) (width 0.2032) (layer F.Cu) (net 7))
 (segment (start 129.8702 37.1602) (end 130.626867 37.1602) (width 0.2032) (layer F.Cu) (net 7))
 (via (at 117.702 38) (size 0.8) (drill 0.4) (layers F.Cu B.Cu) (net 8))
 (via (at 117.7036 40.259) (size 0.8) (drill 0.4) (layers F.Cu B.Cu) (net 8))
 (segment (start 117.702 38) (end 117.629 38) (width 0.2032) (layer F.Cu) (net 8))
 (segment (start 119.225 38) (end 117.702 38) (width 0.2032) (layer F.Cu) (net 8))
 (segment (start 119.126 42.5958) (end 119.126 42.418) (width 0.2032) (layer F.Cu) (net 8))
 (segment (start 117.7036 40.9956) (end 117.7036 40.259) (width 0.2032) (layer F.Cu) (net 8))
 (segment (start 119.126 42.418) (end 117.7036 40.9956) (width 0.2032) (layer F.Cu) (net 8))
 (segment (start 117.702 40.2574) (end 117.7036 40.259) (width 0.2032) (layer B.Cu) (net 8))
 (segment (start 117.702 38) (end 117.702 40.2574) (width 0.2032) (layer B.Cu) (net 8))
 (segment (start 130.029 34.69) (end 130.786 34.69) (width 0.2032) (layer B.Cu) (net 8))
 (segment (start 129.94 34.69) (end 130.786 34.69) (width 0.2032) (layer B.Cu) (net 8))
 (segment (start 128.651 33.401) (end 129.94 34.69) (width 0.2032) (layer B.Cu) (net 8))
 (segment (start 117.702 35.841) (end 120.142 33.401) (width 0.2032) (layer B.Cu) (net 8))
 (segment (start 120.142 33.401) (end 128.651 33.401) (width 0.2032) (layer B.Cu) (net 8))
 (segment (start 117.702 38) (end 117.702 35.841) (width 0.2032) (layer B.Cu) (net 8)))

